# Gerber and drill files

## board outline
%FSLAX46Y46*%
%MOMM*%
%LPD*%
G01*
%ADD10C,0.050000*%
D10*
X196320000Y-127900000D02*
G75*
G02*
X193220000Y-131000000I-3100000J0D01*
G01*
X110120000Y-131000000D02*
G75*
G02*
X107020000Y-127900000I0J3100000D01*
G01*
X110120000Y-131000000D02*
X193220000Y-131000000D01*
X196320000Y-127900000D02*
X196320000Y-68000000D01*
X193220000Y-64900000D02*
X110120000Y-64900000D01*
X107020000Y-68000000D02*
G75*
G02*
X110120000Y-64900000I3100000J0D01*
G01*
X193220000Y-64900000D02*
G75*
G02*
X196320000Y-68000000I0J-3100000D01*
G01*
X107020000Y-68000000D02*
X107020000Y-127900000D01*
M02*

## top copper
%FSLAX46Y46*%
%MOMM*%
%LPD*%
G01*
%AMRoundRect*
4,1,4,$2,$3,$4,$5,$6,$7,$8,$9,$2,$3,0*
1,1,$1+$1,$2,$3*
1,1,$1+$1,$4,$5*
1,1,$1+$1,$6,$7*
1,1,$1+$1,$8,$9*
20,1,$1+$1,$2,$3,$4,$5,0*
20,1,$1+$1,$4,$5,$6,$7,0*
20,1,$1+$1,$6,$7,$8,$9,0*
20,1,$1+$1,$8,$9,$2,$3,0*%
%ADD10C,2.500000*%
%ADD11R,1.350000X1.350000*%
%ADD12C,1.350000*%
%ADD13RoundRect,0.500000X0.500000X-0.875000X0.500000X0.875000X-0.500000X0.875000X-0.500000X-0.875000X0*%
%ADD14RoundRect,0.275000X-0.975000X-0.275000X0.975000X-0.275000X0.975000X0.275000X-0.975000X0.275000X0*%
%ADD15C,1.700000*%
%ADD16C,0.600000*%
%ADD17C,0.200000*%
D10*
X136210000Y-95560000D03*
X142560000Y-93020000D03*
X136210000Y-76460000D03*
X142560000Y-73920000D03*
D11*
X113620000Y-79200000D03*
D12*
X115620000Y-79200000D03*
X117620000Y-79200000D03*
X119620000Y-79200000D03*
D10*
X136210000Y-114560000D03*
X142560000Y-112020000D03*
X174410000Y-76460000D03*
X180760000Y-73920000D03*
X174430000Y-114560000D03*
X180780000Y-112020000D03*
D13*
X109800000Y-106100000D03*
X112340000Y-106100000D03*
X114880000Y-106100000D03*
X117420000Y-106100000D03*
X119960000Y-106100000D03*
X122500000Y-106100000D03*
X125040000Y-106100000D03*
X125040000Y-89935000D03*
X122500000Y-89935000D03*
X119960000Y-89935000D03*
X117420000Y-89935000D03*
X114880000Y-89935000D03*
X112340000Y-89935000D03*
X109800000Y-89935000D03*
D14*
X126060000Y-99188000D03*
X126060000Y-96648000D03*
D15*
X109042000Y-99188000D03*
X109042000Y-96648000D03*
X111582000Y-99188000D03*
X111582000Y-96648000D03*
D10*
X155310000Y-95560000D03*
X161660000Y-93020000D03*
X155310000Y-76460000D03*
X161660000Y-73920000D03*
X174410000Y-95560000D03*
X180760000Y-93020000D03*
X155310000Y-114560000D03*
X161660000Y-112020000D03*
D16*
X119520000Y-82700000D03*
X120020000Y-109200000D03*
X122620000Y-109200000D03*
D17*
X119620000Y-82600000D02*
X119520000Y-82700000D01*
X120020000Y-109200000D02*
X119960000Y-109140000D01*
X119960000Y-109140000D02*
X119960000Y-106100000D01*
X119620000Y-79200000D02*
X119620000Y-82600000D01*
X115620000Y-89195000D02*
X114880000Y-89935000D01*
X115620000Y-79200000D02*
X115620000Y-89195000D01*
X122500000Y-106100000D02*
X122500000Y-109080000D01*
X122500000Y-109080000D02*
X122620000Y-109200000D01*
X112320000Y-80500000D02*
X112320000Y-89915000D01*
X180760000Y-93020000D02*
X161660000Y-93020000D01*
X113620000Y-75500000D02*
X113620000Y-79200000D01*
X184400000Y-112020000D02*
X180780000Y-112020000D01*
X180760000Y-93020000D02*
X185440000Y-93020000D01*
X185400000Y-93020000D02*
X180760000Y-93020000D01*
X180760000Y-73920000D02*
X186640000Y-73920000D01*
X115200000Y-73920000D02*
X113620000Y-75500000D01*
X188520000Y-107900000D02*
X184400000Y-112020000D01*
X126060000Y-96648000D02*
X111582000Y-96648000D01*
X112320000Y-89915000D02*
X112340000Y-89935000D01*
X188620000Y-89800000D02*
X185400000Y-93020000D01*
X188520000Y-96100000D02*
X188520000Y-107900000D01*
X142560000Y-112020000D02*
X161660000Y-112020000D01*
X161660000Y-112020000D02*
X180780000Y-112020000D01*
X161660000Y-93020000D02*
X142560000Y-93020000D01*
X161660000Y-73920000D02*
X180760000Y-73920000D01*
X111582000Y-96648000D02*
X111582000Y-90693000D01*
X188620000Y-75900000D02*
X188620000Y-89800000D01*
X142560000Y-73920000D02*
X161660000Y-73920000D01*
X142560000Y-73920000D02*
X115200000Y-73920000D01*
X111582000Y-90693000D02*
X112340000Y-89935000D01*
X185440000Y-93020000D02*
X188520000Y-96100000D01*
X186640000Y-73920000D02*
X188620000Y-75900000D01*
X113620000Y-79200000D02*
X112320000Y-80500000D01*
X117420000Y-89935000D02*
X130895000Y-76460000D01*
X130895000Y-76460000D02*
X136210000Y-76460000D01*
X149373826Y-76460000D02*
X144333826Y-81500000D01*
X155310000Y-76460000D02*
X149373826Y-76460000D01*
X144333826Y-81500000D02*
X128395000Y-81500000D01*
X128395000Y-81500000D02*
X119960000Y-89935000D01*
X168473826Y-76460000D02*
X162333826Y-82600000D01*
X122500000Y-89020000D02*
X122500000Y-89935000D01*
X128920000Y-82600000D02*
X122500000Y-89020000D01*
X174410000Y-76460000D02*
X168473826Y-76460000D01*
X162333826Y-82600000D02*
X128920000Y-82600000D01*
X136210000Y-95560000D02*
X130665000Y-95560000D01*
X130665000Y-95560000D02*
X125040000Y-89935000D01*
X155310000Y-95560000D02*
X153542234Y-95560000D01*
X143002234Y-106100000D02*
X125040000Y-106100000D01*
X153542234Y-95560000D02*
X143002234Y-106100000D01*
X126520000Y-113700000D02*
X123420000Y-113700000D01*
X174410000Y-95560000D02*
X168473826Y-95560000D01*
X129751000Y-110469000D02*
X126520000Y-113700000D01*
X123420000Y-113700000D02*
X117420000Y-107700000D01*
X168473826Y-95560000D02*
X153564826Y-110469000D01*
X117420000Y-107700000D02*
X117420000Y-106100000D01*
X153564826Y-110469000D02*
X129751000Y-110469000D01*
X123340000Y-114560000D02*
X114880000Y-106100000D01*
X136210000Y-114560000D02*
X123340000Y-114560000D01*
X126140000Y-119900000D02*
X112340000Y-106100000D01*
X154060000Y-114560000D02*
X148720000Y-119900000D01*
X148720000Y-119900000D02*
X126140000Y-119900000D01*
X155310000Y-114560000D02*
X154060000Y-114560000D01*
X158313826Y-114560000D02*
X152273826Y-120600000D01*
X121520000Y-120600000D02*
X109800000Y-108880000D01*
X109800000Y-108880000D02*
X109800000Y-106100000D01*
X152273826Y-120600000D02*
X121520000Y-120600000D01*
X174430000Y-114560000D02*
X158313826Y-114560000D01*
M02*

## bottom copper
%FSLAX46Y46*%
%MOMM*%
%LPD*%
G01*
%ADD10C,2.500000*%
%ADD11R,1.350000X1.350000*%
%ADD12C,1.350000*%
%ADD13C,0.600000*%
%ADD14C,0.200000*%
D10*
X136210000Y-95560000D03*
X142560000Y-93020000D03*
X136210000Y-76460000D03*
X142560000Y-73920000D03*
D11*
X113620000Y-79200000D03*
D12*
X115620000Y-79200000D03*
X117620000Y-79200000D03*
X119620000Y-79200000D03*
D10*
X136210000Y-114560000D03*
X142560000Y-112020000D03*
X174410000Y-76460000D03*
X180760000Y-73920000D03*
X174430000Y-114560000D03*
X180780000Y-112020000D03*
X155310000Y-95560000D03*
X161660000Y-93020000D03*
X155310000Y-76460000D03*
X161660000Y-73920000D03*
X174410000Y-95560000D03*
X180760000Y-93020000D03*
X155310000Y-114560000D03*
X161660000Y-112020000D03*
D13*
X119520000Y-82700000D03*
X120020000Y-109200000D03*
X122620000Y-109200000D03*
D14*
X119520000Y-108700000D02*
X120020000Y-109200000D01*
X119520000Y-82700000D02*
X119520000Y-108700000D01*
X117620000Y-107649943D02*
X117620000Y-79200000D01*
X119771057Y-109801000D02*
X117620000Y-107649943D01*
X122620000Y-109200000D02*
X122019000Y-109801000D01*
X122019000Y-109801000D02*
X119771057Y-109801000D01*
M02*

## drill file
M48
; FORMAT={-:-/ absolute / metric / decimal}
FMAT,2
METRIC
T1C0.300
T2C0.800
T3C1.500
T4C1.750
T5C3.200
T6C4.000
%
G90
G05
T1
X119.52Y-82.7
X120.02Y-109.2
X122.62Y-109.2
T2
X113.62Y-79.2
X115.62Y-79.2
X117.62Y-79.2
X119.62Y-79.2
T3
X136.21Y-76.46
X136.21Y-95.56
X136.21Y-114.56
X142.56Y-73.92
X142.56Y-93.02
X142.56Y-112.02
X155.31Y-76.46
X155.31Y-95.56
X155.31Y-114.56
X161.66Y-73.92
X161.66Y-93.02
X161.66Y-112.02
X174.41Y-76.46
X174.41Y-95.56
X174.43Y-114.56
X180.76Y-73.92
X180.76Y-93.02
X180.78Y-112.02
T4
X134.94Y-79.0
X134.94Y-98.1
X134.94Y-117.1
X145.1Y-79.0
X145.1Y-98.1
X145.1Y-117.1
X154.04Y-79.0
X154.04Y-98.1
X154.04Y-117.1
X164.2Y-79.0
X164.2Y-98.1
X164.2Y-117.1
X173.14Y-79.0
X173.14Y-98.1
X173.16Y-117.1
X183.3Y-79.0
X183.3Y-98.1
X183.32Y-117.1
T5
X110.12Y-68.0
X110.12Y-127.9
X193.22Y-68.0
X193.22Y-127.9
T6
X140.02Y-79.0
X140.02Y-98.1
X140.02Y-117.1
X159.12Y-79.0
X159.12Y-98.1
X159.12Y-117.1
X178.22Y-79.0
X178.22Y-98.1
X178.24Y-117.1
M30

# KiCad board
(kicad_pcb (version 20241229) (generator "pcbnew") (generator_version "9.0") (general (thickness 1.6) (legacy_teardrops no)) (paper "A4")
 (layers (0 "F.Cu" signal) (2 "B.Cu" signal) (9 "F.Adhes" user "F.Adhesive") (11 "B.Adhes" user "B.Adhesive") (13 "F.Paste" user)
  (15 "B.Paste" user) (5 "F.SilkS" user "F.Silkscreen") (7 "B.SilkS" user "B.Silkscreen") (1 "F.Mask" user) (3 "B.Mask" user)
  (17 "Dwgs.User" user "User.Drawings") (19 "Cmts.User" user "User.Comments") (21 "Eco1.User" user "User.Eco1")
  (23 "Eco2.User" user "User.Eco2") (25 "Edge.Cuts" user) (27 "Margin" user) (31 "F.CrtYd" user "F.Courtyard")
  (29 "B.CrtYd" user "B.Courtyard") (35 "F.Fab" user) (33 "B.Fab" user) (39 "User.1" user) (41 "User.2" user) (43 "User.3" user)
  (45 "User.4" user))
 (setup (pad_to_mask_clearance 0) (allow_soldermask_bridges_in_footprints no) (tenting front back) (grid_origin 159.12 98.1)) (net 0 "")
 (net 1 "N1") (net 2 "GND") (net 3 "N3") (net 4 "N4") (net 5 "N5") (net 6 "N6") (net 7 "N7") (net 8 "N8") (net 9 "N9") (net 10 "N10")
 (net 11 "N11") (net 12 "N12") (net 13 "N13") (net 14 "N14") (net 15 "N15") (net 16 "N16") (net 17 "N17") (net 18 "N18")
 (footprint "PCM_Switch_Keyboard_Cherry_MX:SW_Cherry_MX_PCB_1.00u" (layer "F.Cu") (at 140.02 98.1)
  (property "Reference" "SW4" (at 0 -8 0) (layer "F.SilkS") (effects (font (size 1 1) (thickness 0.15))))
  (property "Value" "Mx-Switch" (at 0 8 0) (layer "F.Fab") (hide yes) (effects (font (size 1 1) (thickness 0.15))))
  (pad "" np_thru_hole circle (at -5.08 0) (size 1.75 1.75) (drill 1.75) (layers "*.Cu" "*.Mask"))
  (pad "" np_thru_hole circle (at 0 0) (size 4 4) (drill 4) (layers "*.Cu" "*.Mask"))
  (pad "" np_thru_hole circle (at 5.08 0) (size 1.75 1.75) (drill 1.75) (layers "*.Cu" "*.Mask"))
  (pad "1" thru_hole circle (at -3.81 -2.54) (size 2.5 2.5) (drill 1.5) (layers "*.Cu" "*.Mask") (remove_unused_layers no) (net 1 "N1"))
  (pad "2" thru_hole circle (at 2.54 -5.08) (size 2.5 2.5) (drill 1.5) (layers "*.Cu" "*.Mask") (remove_unused_layers no) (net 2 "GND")))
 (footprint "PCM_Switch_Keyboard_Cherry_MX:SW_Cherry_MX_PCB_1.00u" (layer "F.Cu") (at 140.02 79)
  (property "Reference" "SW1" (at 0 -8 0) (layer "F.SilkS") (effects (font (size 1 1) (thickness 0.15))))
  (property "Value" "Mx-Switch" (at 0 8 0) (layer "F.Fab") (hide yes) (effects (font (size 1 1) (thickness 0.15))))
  (pad "" np_thru_hole circle (at -5.08 0) (size 1.75 1.75) (drill 1.75) (layers "*.Cu" "*.Mask"))
  (pad "" np_thru_hole circle (at 0 0) (size 4 4) (drill 4) (layers "*.Cu" "*.Mask"))
  (pad "" np_thru_hole circle (at 5.08 0) (size 1.75 1.75) (drill 1.75) (layers "*.Cu" "*.Mask"))
  (pad "1" thru_hole circle (at -3.81 -2.54) (size 2.5 2.5) (drill 1.5) (layers "*.Cu" "*.Mask") (remove_unused_layers no) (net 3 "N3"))
  (pad "2" thru_hole circle (at 2.54 -5.08) (size 2.5 2.5) (drill 1.5) (layers "*.Cu" "*.Mask") (remove_unused_layers no) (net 2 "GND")))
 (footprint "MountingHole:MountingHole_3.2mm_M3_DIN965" (layer "F.Cu") (at 193.22 68)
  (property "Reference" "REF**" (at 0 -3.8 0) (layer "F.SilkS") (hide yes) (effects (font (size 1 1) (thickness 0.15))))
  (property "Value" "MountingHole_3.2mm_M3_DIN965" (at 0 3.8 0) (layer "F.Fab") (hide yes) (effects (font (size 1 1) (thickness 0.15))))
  (pad "" np_thru_hole circle (at 0 0) (size 3.2 3.2) (drill 3.2) (layers "*.Cu" "*.Mask")))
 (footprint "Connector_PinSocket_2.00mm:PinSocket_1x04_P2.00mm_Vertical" (layer "F.Cu") (at 113.62 79.2 90)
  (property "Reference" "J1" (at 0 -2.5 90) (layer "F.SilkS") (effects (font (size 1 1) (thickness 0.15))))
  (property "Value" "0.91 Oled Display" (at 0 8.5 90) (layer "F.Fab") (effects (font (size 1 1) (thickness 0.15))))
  (pad "1" thru_hole rect (at 0 0 90) (size 1.35 1.35) (drill 0.8) (layers "*.Cu" "*.Mask") (remove_unused_layers no) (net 2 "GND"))
  (pad "2" thru_hole circle (at 0 2 90) (size 1.35 1.35) (drill 0.8) (layers "*.Cu" "*.Mask") (remove_unused_layers no) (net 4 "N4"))
  (pad "3" thru_hole circle (at 0 4 90) (size 1.35 1.35) (drill 0.8) (layers "*.Cu" "*.Mask") (remove_unused_layers no) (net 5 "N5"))
  (pad "4" thru_hole circle (at 0 6 90) (size 1.35 1.35) (drill 0.8) (layers "*.Cu" "*.Mask") (remove_unused_layers no) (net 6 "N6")))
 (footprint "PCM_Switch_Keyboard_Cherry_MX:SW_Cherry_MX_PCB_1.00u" (layer "F.Cu") (at 140.02 117.1)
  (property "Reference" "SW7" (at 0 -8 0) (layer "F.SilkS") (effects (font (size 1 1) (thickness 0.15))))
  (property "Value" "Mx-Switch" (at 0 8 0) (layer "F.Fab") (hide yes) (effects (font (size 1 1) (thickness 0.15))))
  (pad "" np_thru_hole circle (at -5.08 0) (size 1.75 1.75) (drill 1.75) (layers "*.Cu" "*.Mask"))
  (pad "" np_thru_hole circle (at 0 0) (size 4 4) (drill 4) (layers "*.Cu" "*.Mask"))
  (pad "" np_thru_hole circle (at 5.08 0) (size 1.75 1.75) (drill 1.75) (layers "*.Cu" "*.Mask"))
  (pad "1" thru_hole circle (at -3.81 -2.54) (size 2.5 2.5) (drill 1.5) (layers "*.Cu" "*.Mask") (remove_unused_layers no) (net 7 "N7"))
  (pad "2" thru_hole circle (at 2.54 -5.08) (size 2.5 2.5) (drill 1.5) (layers "*.Cu" "*.Mask") (remove_unused_layers no) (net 2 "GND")))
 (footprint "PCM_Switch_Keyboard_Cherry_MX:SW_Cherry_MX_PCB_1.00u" (layer "F.Cu") (at 178.22 79)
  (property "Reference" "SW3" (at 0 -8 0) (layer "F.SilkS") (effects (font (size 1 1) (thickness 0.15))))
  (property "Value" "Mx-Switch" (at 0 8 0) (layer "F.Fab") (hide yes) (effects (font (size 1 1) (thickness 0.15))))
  (pad "" np_thru_hole circle (at -5.08 0) (size 1.75 1.75) (drill 1.75) (layers "*.Cu" "*.Mask"))
  (pad "" np_thru_hole circle (at 0 0) (size 4 4) (drill 4) (layers "*.Cu" "*.Mask"))
  (pad "" np_thru_hole circle (at 5.08 0) (size 1.75 1.75) (drill 1.75) (layers "*.Cu" "*.Mask"))
  (pad "1" thru_hole circle (at -3.81 -2.54) (size 2.5 2.5) (drill 1.5) (layers "*.Cu" "*.Mask") (remove_unused_layers no) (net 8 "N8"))
  (pad "2" thru_hole circle (at 2.54 -5.08) (size 2.5 2.5) (drill 1.5) (layers "*.Cu" "*.Mask") (remove_unused_layers no) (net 2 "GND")))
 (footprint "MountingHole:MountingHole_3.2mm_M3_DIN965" (layer "F.Cu") (at 110.12 68)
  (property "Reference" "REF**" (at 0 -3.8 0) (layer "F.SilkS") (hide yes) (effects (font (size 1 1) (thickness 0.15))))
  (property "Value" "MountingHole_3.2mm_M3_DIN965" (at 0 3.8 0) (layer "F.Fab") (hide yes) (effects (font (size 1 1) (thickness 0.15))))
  (pad "" np_thru_hole circle (at 0 0) (size 3.2 3.2) (drill 3.2) (layers "*.Cu" "*.Mask")))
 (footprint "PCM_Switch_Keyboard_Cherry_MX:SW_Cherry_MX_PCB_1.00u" (layer "F.Cu") (at 178.24 117.1)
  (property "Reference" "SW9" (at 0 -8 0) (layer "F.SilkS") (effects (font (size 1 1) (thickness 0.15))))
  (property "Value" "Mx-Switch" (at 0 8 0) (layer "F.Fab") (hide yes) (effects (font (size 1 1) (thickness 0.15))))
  (pad "" np_thru_hole circle (at -5.08 0) (size 1.75 1.75) (drill 1.75) (layers "*.Cu" "*.Mask"))
  (pad "" np_thru_hole circle (at 0 0) (size 4 4) (drill 4) (layers "*.Cu" "*.Mask"))
  (pad "" np_thru_hole circle (at 5.08 0) (size 1.75 1.75) (drill 1.75) (layers "*.Cu" "*.Mask"))
  (pad "1" thru_hole circle (at -3.81 -2.54) (size 2.5 2.5) (drill 1.5) (layers "*.Cu" "*.Mask") (remove_unused_layers no) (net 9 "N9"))
  (pad "2" thru_hole circle (at 2.54 -5.08) (size 2.5 2.5) (drill 1.5) (layers "*.Cu" "*.Mask") (remove_unused_layers no) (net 2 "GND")))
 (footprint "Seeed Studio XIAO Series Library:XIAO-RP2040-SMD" (layer "F.Cu") (at 117.42 98.1 90)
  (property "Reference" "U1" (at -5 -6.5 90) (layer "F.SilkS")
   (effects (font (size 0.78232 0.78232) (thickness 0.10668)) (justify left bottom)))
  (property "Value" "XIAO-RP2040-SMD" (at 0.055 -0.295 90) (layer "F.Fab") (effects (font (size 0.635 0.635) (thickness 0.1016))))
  (pad "1" smd roundrect (at -8 -7.62 90) (size 2.75 2) (layers "F.Cu" "F.Mask" "F.Paste") (roundrect_rratio 0.25) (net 9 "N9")
   (solder_mask_margin 0.0508) (thermal_bridge_angle 45))
  (pad "2" smd roundrect (at -8 -5.08 90) (size 2.75 2) (layers "F.Cu" "F.Mask" "F.Paste") (roundrect_rratio 0.25) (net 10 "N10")
   (solder_mask_margin 0.0508) (thermal_bridge_angle 45))
  (pad "3" smd roundrect (at -8 -2.54 90) (size 2.75 2) (layers "F.Cu" "F.Mask" "F.Paste") (roundrect_rratio 0.25) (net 7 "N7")
   (solder_mask_margin 0.0508) (thermal_bridge_angle 45))
  (pad "4" smd roundrect (at -8 0 90) (size 2.75 2) (layers "F.Cu" "F.Mask" "F.Paste") (roundrect_rratio 0.25) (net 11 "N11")
   (solder_mask_margin 0.0508) (thermal_bridge_angle 45))
  (pad "5" smd roundrect (at -8 2.54 90) (size 2.75 2) (layers "F.Cu" "F.Mask" "F.Paste") (roundrect_rratio 0.25) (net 6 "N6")
   (solder_mask_margin 0.0508) (thermal_bridge_angle 45))
  (pad "6" smd roundrect (at -8 5.08 90) (size 2.75 2) (layers "F.Cu" "F.Mask" "F.Paste") (roundrect_rratio 0.25) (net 5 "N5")
   (solder_mask_margin 0.0508) (thermal_bridge_angle 45))
  (pad "7" smd roundrect (at -8 7.62 90) (size 2.75 2) (layers "F.Cu" "F.Mask" "F.Paste") (roundrect_rratio 0.25) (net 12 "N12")
   (solder_mask_margin 0.0508) (thermal_bridge_angle 45))
  (pad "8" smd roundrect (at 8.165 7.62 90) (size 2.75 2) (layers "F.Cu" "F.Mask" "F.Paste") (roundrect_rratio 0.25) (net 1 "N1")
   (solder_mask_margin 0.0508) (thermal_bridge_angle 45))
  (pad "9" smd roundrect (at 8.165 5.08 90) (size 2.75 2) (layers "F.Cu" "F.Mask" "F.Paste") (roundrect_rratio 0.25) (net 8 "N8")
   (solder_mask_margin 0.0508) (thermal_bridge_angle 45))
  (pad "10" smd roundrect (at 8.165 2.54 90) (size 2.75 2) (layers "F.Cu" "F.Mask" "F.Paste") (roundrect_rratio 0.25) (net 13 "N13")
   (solder_mask_margin 0.0508) (thermal_bridge_angle 45))
  (pad "11" smd roundrect (at 8.165 0 90) (size 2.75 2) (layers "F.Cu" "F.Mask" "F.Paste") (roundrect_rratio 0.25) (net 3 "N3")
   (solder_mask_margin 0.0508) (thermal_bridge_angle 45))
  (pad "12" smd roundrect (at 8.165 -2.54 90) (size 2.75 2) (layers "F.Cu" "F.Mask" "F.Paste") (roundrect_rratio 0.25) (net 4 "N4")
   (solder_mask_margin 0.0508) (thermal_bridge_angle 45))
  (pad "13" smd roundrect (at 8.165 -5.08 90) (size 2.75 2) (layers "F.Cu" "F.Mask" "F.Paste") (roundrect_rratio 0.25) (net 2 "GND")
   (solder_mask_margin 0.0508) (thermal_bridge_angle 45))
  (pad "14" smd roundrect (at 8.165 -7.62 90) (size 2.75 2) (layers "F.Cu" "F.Mask" "F.Paste") (roundrect_rratio 0.25) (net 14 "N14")
   (solder_mask_margin 0.0508) (thermal_bridge_angle 45))
  (pad "15" smd roundrect (at -1.088 8.64) (size 2.5 1.1) (layers "F.Cu" "F.Mask" "F.Paste") (roundrect_rratio 0.25) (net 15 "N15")
   (thermal_bridge_angle 45))
  (pad "16" smd roundrect (at 1.452 8.64) (size 2.5 1.1) (layers "F.Cu" "F.Mask" "F.Paste") (roundrect_rratio 0.25) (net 2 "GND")
   (thermal_bridge_angle 45))
  (pad "17" smd circle (at -1.088 -8.378 90) (size 1.7 1.7) (layers "F.Cu" "F.Mask" "F.Paste") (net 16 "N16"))
  (pad "18" smd circle (at 1.452 -8.378 90) (size 1.7 1.7) (layers "F.Cu" "F.Mask" "F.Paste") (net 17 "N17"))
  (pad "19" smd circle (at -1.088 -5.838 90) (size 1.7 1.7) (layers "F.Cu" "F.Mask" "F.Paste") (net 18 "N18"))
  (pad "20" smd circle (at 1.452 -5.838 90) (size 1.7 1.7) (layers "F.Cu" "F.Mask" "F.Paste") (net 2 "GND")))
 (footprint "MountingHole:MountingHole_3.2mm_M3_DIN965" (layer "F.Cu") (at 110.12 127.9)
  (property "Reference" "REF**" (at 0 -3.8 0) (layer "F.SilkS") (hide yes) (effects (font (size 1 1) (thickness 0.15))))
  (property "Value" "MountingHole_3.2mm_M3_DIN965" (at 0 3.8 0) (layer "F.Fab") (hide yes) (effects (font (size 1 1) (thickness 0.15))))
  (pad "" np_thru_hole circle (at 0 0) (size 3.2 3.2) (drill 3.2) (layers "*.Cu" "*.Mask")))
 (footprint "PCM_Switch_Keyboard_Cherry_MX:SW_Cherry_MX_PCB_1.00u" (layer "F.Cu") (at 159.12 98.1)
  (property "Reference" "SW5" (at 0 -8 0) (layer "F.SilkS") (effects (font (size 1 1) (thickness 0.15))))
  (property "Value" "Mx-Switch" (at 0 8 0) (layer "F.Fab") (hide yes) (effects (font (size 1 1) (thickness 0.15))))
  (pad "" np_thru_hole circle (at -5.08 0) (size 1.75 1.75) (drill 1.75) (layers "*.Cu" "*.Mask"))
  (pad "" np_thru_hole circle (at 0 0) (size 4 4) (drill 4) (layers "*.Cu" "*.Mask"))
  (pad "" np_thru_hole circle (at 5.08 0) (size 1.75 1.75) (drill 1.75) (layers "*.Cu" "*.Mask"))
  (pad "1" thru_hole circle (at -3.81 -2.54) (size 2.5 2.5) (drill 1.5) (layers "*.Cu" "*.Mask") (remove_unused_layers no) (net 12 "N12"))
  (pad "2" thru_hole circle (at 2.54 -5.08) (size 2.5 2.5) (drill 1.5) (layers "*.Cu" "*.Mask") (remove_unused_layers no) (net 2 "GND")))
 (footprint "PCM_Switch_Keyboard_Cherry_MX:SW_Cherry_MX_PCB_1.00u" (layer "F.Cu") (at 159.12 79)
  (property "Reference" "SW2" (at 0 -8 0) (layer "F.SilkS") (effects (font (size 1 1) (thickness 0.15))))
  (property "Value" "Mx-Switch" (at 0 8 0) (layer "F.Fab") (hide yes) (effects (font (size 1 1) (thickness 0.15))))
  (pad "" np_thru_hole circle (at -5.08 0) (size 1.75 1.75) (drill 1.75) (layers "*.Cu" "*.Mask"))
  (pad "" np_thru_hole circle (at 0 0) (size 4 4) (drill 4) (layers "*.Cu" "*.Mask"))
  (pad "" np_thru_hole circle (at 5.08 0) (size 1.75 1.75) (drill 1.75) (layers "*.Cu" "*.Mask"))
  (pad "1" thru_hole circle (at -3.81 -2.54) (size 2.5 2.5) (drill 1.5) (layers "*.Cu" "*.Mask") (remove_unused_layers no) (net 13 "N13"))
  (pad "2" thru_hole circle (at 2.54 -5.08) (size 2.5 2.5) (drill 1.5) (layers "*.Cu" "*.Mask") (remove_unused_layers no) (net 2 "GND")))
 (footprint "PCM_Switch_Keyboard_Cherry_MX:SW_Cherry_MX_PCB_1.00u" (layer "F.Cu") (at 178.22 98.1)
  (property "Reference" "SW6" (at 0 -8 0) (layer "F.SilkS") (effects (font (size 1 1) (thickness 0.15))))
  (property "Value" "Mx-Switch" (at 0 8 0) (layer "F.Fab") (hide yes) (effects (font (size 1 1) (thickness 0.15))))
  (pad "" np_thru_hole circle (at -5.08 0) (size 1.75 1.75) (drill 1.75) (layers "*.Cu" "*.Mask"))
  (pad "" np_thru_hole circle (at 0 0) (size 4 4) (drill 4) (layers "*.Cu" "*.Mask"))
  (pad "" np_thru_hole circle (at 5.08 0) (size 1.75 1.75) (drill 1.75) (layers "*.Cu" "*.Mask"))
  (pad "1" thru_hole circle (at -3.81 -2.54) (size 2.5 2.5) (drill 1.5) (layers "*.Cu" "*.Mask") (remove_unused_layers no) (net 11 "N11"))
  (pad "2" thru_hole circle (at 2.54 -5.08) (size 2.5 2.5) (drill 1.5) (layers "*.Cu" "*.Mask") (remove_unused_layers no) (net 2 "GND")))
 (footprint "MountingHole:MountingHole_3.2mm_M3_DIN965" (layer "F.Cu") (at 193.22 127.9)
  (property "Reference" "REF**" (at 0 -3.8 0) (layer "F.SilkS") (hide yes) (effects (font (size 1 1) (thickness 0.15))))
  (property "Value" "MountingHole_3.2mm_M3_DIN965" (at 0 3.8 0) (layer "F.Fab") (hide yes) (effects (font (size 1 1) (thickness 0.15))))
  (pad "" np_thru_hole circle (at 0 0) (size 3.2 3.2) (drill 3.2) (layers "*.Cu" "*.Mask")))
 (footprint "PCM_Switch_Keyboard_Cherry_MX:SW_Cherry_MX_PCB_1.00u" (layer "F.Cu") (at 159.12 117.1)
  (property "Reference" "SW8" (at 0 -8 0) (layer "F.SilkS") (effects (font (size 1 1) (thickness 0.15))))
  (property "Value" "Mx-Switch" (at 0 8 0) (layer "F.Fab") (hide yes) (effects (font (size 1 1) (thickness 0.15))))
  (pad "" np_thru_hole circle (at -5.08 0) (size 1.75 1.75) (drill 1.75) (layers "*.Cu" "*.Mask"))
  (pad "" np_thru_hole circle (at 0 0) (size 4 4) (drill 4) (layers "*.Cu" "*.Mask"))
  (pad "" np_thru_hole circle (at 5.08 0) (size 1.75 1.75) (drill 1.75) (layers "*.Cu" "*.Mask"))
  (pad "1" thru_hole circle (at -3.81 -2.54) (size 2.5 2.5) (drill 1.5) (layers "*.Cu" "*.Mask") (remove_unused_layers no) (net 10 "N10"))
  (pad "2" thru_hole circle (at 2.54 -5.08) (size 2.5 2.5) (drill 1.5) (layers "*.Cu" "*.Mask") (remove_unused_layers no) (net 2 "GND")))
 (gr_arc (start 196.32 127.9) (mid 195.412031 130.092031) (end 193.22 131) (stroke (width 0.05) (type default)) (layer "Edge.Cuts"))
 (gr_arc (start 110.12 131) (mid 107.927969 130.092031) (end 107.02 127.9) (stroke (width 0.05) (type default)) (layer "Edge.Cuts"))
 (gr_line (start 110.12 131) (end 193.22 131) (stroke (width 0.05) (type default)) (layer "Edge.Cuts"))
 (gr_line (start 196.32 127.9) (end 196.32 68) (stroke (width 0.05) (type default)) (layer "Edge.Cuts"))
 (gr_line (start 193.22 64.9) (end 110.12 64.9) (stroke (width 0.05) (type default)) (layer "Edge.Cuts"))
 (gr_arc (start 107.02 68) (mid 107.927969 65.807969) (end 110.12 64.9) (stroke (width 0.05) (type solid)) (layer "Edge.Cuts"))
 (gr_arc (start 193.22 64.9) (mid 195.412031 65.807969) (end 196.32 68) (stroke (width 0.05) (type default)) (layer "Edge.Cuts"))
 (gr_line (start 107.02 68) (end 107.02 127.9) (stroke (width 0.05) (type default)) (layer "Edge.Cuts"))
 (segment (start 119.62 82.6) (end 119.52 82.7) (width 0.2) (layer "F.Cu") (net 6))
 (segment (start 120.02 109.2) (end 119.96 109.14) (width 0.2) (layer "F.Cu") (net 6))
 (segment (start 119.96 109.14) (end 119.96 106.1) (width 0.2) (layer "F.Cu") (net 6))
 (segment (start 119.62 79.2) (end 119.62 82.6) (width 0.2) (layer "F.Cu") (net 6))
 (via (at 119.52 82.7) (size 0.6) (drill 0.3) (layers "F.Cu" "B.Cu") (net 6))
 (via (at 120.02 109.2) (size 0.6) (drill 0.3) (layers "F.Cu" "B.Cu") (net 6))
 (segment (start 119.52 108.7) (end 120.02 109.2) (width 0.2) (layer "B.Cu") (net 6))
 (segment (start 119.52 82.7) (end 119.52 108.7) (width 0.2) (layer "B.Cu") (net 6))
 (segment (start 115.62 89.195) (end 114.88 89.935) (width 0.2) (layer "F.Cu") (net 4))
 (segment (start 115.62 79.2) (end 115.62 89.195) (width 0.2) (layer "F.Cu") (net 4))
 (segment (start 122.5 106.1) (end 122.5 109.08) (width 0.2) (layer "F.Cu") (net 5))
 (segment (start 122.5 109.08) (end 122.62 109.2) (width 0.2) (layer "F.Cu") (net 5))
 (via (at 122.62 109.2) (size 0.6) (drill 0.3) (layers "F.Cu" "B.Cu") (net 5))
 (segment (start 117.62 107.649943) (end 117.62 79.2) (width 0.2) (layer "B.Cu") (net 5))
 (segment (start 119.771057 109.801) (end 117.62 107.649943) (width 0.2) (layer "B.Cu") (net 5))
 (segment (start 122.62 109.2) (end 122.019 109.801) (width 0.2) (layer "B.Cu") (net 5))
 (segment (start 122.019 109.801) (end 119.771057 109.801) (width 0.2) (layer "B.Cu") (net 5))
 (segment (start 112.32 80.5) (end 112.32 89.915) (width 0.2) (layer "F.Cu") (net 2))
 (segment (start 180.76 93.02) (end 161.66 93.02) (width 0.2) (layer "F.Cu") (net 2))
 (segment (start 113.62 75.5) (end 113.62 79.2) (width 0.2) (layer "F.Cu") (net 2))
 (segment (start 184.4 112.02) (end 180.78 112.02) (width 0.2) (layer "F.Cu") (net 2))
 (segment (start 180.76 93.02) (end 185.44 93.02) (width 0.2) (layer "F.Cu") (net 2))
 (segment (start 185.4 93.02) (end 180.76 93.02) (width 0.2) (layer "F.Cu") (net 2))
 (segment (start 180.76 73.92) (end 186.64 73.92) (width 0.2) (layer "F.Cu") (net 2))
 (segment (start 115.2 73.92) (end 113.62 75.5) (width 0.2) (layer "F.Cu") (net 2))
 (segment (start 188.52 107.9) (end 184.4 112.02) (width 0.2) (layer "F.Cu") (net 2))
 (segment (start 126.06 96.648) (end 111.582 96.648) (width 0.2) (layer "F.Cu") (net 2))
 (segment (start 112.32 89.915) (end 112.34 89.935) (width 0.2) (layer "F.Cu") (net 2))
 (segment (start 188.62 89.8) (end 185.4 93.02) (width 0.2) (layer "F.Cu") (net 2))
 (segment (start 188.52 96.1) (end 188.52 107.9) (width 0.2) (layer "F.Cu") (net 2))
 (segment (start 142.56 112.02) (end 161.66 112.02) (width 0.2) (layer "F.Cu") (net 2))
 (segment (start 161.66 112.02) (end 180.78 112.02) (width 0.2) (layer "F.Cu") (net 2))
 (segment (start 161.66 93.02) (end 142.56 93.02) (width 0.2) (layer "F.Cu") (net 2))
 (segment (start 161.66 73.92) (end 180.76 73.92) (width 0.2) (layer "F.Cu") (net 2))
 (segment (start 111.582 96.648) (end 111.582 90.693) (width 0.2) (layer "F.Cu") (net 2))
 (segment (start 188.62 75.9) (end 188.62 89.8) (width 0.2) (layer "F.Cu") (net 2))
 (segment (start 142.56 73.92) (end 161.66 73.92) (width 0.2) (layer "F.Cu") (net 2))
 (segment (start 142.56 73.92) (end 115.2 73.92) (width 0.2) (layer "F.Cu") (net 2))
 (segment (start 111.582 90.693) (end 112.34 89.935) (width 0.2) (layer "F.Cu") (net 2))
 (segment (start 185.44 93.02) (end 188.52 96.1) (width 0.2) (layer "F.Cu") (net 2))
 (segment (start 186.64 73.92) (end 188.62 75.9) (width 0.2) (layer "F.Cu") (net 2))
 (segment (start 113.62 79.2) (end 112.32 80.5) (width 0.2) (layer "F.Cu") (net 2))
 (segment (start 117.42 89.935) (end 130.895 76.46) (width 0.2) (layer "F.Cu") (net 3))
 (segment (start 130.895 76.46) (end 136.21 76.46) (width 0.2) (layer "F.Cu") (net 3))
 (segment (start 149.373826 76.46) (end 144.333826 81.5) (width 0.2) (layer "F.Cu") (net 13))
 (segment (start 155.31 76.46) (end 149.373826 76.46) (width 0.2) (layer "F.Cu") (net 13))
 (segment (start 144.333826 81.5) (end 128.395 81.5) (width 0.2) (layer "F.Cu") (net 13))
 (segment (start 128.395 81.5) (end 119.96 89.935) (width 0.2) (layer "F.Cu") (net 13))
 (segment (start 168.473826 76.46) (end 162.333826 82.6) (width 0.2) (layer "F.Cu") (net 8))
 (segment (start 122.5 89.02) (end 122.5 89.935) (width 0.2) (layer "F.Cu") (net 8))
 (segment (start 128.92 82.6) (end 122.5 89.02) (width 0.2) (layer "F.Cu") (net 8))
 (segment (start 174.41 76.46) (end 168.473826 76.46) (width 0.2) (layer "F.Cu") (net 8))
 (segment (start 162.333826 82.6) (end 128.92 82.6) (width 0.2) (layer "F.Cu") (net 8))
 (segment (start 136.21 95.56) (end 130.665 95.56) (width 0.2) (layer "F.Cu") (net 1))
 (segment (start 130.665 95.56) (end 125.04 89.935) (width 0.2) (layer "F.Cu") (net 1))
 (segment (start 155.31 95.56) (end 153.542234 95.56) (width 0.2) (layer "F.Cu") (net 12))
 (segment (start 143.002234 106.1) (end 125.04 106.1) (width 0.2) (layer "F.Cu") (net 12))
 (segment (start 153.542234 95.56) (end 143.002234 106.1) (width 0.2) (layer "F.Cu") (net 12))
 (segment (start 126.52 113.7) (end 123.42 113.7) (width 0.2) (layer "F.Cu") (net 11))
 (segment (start 174.41 95.56) (end 168.473826 95.56) (width 0.2) (layer "F.Cu") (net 11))
 (segment (start 129.751 110.469) (end 126.52 113.7) (width 0.2) (layer "F.Cu") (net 11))
 (segment (start 123.42 113.7) (end 117.42 107.7) (width 0.2) (layer "F.Cu") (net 11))
 (segment (start 168.473826 95.56) (end 153.564826 110.469) (width 0.2) (layer "F.Cu") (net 11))
 (segment (start 117.42 107.7) (end 117.42 106.1) (width 0.2) (layer "F.Cu") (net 11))
 (segment (start 153.564826 110.469) (end 129.751 110.469) (width 0.2) (layer "F.Cu") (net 11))
 (segment (start 123.34 114.56) (end 114.88 106.1) (width 0.2) (layer "F.Cu") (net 7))
 (segment (start 136.21 114.56) (end 123.34 114.56) (width 0.2) (layer "F.Cu") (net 7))
 (segment (start 126.14 119.9) (end 112.34 106.1) (width 0.2) (layer "F.Cu") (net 10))
 (segment (start 154.06 114.56) (end 148.72 119.9) (width 0.2) (layer "F.Cu") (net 10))
 (segment (start 148.72 119.9) (end 126.14 119.9) (width 0.2) (layer "F.Cu") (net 10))
 (segment (start 155.31 114.56) (end 154.06 114.56) (width 0.2) (layer "F.Cu") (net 10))
 (segment (start 158.313826 114.56) (end 152.273826 120.6) (width 0.2) (layer "F.Cu") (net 9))
 (segment (start 121.52 120.6) (end 109.8 108.88) (width 0.2) (layer "F.Cu") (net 9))
 (segment (start 109.8 108.88) (end 109.8 106.1) (width 0.2) (layer "F.Cu") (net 9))
 (segment (start 152.273826 120.6) (end 121.52 120.6) (width 0.2) (layer "F.Cu") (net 9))
 (segment (start 174.43 114.56) (end 158.313826 114.56) (width 0.2) (layer "F.Cu") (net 9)))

